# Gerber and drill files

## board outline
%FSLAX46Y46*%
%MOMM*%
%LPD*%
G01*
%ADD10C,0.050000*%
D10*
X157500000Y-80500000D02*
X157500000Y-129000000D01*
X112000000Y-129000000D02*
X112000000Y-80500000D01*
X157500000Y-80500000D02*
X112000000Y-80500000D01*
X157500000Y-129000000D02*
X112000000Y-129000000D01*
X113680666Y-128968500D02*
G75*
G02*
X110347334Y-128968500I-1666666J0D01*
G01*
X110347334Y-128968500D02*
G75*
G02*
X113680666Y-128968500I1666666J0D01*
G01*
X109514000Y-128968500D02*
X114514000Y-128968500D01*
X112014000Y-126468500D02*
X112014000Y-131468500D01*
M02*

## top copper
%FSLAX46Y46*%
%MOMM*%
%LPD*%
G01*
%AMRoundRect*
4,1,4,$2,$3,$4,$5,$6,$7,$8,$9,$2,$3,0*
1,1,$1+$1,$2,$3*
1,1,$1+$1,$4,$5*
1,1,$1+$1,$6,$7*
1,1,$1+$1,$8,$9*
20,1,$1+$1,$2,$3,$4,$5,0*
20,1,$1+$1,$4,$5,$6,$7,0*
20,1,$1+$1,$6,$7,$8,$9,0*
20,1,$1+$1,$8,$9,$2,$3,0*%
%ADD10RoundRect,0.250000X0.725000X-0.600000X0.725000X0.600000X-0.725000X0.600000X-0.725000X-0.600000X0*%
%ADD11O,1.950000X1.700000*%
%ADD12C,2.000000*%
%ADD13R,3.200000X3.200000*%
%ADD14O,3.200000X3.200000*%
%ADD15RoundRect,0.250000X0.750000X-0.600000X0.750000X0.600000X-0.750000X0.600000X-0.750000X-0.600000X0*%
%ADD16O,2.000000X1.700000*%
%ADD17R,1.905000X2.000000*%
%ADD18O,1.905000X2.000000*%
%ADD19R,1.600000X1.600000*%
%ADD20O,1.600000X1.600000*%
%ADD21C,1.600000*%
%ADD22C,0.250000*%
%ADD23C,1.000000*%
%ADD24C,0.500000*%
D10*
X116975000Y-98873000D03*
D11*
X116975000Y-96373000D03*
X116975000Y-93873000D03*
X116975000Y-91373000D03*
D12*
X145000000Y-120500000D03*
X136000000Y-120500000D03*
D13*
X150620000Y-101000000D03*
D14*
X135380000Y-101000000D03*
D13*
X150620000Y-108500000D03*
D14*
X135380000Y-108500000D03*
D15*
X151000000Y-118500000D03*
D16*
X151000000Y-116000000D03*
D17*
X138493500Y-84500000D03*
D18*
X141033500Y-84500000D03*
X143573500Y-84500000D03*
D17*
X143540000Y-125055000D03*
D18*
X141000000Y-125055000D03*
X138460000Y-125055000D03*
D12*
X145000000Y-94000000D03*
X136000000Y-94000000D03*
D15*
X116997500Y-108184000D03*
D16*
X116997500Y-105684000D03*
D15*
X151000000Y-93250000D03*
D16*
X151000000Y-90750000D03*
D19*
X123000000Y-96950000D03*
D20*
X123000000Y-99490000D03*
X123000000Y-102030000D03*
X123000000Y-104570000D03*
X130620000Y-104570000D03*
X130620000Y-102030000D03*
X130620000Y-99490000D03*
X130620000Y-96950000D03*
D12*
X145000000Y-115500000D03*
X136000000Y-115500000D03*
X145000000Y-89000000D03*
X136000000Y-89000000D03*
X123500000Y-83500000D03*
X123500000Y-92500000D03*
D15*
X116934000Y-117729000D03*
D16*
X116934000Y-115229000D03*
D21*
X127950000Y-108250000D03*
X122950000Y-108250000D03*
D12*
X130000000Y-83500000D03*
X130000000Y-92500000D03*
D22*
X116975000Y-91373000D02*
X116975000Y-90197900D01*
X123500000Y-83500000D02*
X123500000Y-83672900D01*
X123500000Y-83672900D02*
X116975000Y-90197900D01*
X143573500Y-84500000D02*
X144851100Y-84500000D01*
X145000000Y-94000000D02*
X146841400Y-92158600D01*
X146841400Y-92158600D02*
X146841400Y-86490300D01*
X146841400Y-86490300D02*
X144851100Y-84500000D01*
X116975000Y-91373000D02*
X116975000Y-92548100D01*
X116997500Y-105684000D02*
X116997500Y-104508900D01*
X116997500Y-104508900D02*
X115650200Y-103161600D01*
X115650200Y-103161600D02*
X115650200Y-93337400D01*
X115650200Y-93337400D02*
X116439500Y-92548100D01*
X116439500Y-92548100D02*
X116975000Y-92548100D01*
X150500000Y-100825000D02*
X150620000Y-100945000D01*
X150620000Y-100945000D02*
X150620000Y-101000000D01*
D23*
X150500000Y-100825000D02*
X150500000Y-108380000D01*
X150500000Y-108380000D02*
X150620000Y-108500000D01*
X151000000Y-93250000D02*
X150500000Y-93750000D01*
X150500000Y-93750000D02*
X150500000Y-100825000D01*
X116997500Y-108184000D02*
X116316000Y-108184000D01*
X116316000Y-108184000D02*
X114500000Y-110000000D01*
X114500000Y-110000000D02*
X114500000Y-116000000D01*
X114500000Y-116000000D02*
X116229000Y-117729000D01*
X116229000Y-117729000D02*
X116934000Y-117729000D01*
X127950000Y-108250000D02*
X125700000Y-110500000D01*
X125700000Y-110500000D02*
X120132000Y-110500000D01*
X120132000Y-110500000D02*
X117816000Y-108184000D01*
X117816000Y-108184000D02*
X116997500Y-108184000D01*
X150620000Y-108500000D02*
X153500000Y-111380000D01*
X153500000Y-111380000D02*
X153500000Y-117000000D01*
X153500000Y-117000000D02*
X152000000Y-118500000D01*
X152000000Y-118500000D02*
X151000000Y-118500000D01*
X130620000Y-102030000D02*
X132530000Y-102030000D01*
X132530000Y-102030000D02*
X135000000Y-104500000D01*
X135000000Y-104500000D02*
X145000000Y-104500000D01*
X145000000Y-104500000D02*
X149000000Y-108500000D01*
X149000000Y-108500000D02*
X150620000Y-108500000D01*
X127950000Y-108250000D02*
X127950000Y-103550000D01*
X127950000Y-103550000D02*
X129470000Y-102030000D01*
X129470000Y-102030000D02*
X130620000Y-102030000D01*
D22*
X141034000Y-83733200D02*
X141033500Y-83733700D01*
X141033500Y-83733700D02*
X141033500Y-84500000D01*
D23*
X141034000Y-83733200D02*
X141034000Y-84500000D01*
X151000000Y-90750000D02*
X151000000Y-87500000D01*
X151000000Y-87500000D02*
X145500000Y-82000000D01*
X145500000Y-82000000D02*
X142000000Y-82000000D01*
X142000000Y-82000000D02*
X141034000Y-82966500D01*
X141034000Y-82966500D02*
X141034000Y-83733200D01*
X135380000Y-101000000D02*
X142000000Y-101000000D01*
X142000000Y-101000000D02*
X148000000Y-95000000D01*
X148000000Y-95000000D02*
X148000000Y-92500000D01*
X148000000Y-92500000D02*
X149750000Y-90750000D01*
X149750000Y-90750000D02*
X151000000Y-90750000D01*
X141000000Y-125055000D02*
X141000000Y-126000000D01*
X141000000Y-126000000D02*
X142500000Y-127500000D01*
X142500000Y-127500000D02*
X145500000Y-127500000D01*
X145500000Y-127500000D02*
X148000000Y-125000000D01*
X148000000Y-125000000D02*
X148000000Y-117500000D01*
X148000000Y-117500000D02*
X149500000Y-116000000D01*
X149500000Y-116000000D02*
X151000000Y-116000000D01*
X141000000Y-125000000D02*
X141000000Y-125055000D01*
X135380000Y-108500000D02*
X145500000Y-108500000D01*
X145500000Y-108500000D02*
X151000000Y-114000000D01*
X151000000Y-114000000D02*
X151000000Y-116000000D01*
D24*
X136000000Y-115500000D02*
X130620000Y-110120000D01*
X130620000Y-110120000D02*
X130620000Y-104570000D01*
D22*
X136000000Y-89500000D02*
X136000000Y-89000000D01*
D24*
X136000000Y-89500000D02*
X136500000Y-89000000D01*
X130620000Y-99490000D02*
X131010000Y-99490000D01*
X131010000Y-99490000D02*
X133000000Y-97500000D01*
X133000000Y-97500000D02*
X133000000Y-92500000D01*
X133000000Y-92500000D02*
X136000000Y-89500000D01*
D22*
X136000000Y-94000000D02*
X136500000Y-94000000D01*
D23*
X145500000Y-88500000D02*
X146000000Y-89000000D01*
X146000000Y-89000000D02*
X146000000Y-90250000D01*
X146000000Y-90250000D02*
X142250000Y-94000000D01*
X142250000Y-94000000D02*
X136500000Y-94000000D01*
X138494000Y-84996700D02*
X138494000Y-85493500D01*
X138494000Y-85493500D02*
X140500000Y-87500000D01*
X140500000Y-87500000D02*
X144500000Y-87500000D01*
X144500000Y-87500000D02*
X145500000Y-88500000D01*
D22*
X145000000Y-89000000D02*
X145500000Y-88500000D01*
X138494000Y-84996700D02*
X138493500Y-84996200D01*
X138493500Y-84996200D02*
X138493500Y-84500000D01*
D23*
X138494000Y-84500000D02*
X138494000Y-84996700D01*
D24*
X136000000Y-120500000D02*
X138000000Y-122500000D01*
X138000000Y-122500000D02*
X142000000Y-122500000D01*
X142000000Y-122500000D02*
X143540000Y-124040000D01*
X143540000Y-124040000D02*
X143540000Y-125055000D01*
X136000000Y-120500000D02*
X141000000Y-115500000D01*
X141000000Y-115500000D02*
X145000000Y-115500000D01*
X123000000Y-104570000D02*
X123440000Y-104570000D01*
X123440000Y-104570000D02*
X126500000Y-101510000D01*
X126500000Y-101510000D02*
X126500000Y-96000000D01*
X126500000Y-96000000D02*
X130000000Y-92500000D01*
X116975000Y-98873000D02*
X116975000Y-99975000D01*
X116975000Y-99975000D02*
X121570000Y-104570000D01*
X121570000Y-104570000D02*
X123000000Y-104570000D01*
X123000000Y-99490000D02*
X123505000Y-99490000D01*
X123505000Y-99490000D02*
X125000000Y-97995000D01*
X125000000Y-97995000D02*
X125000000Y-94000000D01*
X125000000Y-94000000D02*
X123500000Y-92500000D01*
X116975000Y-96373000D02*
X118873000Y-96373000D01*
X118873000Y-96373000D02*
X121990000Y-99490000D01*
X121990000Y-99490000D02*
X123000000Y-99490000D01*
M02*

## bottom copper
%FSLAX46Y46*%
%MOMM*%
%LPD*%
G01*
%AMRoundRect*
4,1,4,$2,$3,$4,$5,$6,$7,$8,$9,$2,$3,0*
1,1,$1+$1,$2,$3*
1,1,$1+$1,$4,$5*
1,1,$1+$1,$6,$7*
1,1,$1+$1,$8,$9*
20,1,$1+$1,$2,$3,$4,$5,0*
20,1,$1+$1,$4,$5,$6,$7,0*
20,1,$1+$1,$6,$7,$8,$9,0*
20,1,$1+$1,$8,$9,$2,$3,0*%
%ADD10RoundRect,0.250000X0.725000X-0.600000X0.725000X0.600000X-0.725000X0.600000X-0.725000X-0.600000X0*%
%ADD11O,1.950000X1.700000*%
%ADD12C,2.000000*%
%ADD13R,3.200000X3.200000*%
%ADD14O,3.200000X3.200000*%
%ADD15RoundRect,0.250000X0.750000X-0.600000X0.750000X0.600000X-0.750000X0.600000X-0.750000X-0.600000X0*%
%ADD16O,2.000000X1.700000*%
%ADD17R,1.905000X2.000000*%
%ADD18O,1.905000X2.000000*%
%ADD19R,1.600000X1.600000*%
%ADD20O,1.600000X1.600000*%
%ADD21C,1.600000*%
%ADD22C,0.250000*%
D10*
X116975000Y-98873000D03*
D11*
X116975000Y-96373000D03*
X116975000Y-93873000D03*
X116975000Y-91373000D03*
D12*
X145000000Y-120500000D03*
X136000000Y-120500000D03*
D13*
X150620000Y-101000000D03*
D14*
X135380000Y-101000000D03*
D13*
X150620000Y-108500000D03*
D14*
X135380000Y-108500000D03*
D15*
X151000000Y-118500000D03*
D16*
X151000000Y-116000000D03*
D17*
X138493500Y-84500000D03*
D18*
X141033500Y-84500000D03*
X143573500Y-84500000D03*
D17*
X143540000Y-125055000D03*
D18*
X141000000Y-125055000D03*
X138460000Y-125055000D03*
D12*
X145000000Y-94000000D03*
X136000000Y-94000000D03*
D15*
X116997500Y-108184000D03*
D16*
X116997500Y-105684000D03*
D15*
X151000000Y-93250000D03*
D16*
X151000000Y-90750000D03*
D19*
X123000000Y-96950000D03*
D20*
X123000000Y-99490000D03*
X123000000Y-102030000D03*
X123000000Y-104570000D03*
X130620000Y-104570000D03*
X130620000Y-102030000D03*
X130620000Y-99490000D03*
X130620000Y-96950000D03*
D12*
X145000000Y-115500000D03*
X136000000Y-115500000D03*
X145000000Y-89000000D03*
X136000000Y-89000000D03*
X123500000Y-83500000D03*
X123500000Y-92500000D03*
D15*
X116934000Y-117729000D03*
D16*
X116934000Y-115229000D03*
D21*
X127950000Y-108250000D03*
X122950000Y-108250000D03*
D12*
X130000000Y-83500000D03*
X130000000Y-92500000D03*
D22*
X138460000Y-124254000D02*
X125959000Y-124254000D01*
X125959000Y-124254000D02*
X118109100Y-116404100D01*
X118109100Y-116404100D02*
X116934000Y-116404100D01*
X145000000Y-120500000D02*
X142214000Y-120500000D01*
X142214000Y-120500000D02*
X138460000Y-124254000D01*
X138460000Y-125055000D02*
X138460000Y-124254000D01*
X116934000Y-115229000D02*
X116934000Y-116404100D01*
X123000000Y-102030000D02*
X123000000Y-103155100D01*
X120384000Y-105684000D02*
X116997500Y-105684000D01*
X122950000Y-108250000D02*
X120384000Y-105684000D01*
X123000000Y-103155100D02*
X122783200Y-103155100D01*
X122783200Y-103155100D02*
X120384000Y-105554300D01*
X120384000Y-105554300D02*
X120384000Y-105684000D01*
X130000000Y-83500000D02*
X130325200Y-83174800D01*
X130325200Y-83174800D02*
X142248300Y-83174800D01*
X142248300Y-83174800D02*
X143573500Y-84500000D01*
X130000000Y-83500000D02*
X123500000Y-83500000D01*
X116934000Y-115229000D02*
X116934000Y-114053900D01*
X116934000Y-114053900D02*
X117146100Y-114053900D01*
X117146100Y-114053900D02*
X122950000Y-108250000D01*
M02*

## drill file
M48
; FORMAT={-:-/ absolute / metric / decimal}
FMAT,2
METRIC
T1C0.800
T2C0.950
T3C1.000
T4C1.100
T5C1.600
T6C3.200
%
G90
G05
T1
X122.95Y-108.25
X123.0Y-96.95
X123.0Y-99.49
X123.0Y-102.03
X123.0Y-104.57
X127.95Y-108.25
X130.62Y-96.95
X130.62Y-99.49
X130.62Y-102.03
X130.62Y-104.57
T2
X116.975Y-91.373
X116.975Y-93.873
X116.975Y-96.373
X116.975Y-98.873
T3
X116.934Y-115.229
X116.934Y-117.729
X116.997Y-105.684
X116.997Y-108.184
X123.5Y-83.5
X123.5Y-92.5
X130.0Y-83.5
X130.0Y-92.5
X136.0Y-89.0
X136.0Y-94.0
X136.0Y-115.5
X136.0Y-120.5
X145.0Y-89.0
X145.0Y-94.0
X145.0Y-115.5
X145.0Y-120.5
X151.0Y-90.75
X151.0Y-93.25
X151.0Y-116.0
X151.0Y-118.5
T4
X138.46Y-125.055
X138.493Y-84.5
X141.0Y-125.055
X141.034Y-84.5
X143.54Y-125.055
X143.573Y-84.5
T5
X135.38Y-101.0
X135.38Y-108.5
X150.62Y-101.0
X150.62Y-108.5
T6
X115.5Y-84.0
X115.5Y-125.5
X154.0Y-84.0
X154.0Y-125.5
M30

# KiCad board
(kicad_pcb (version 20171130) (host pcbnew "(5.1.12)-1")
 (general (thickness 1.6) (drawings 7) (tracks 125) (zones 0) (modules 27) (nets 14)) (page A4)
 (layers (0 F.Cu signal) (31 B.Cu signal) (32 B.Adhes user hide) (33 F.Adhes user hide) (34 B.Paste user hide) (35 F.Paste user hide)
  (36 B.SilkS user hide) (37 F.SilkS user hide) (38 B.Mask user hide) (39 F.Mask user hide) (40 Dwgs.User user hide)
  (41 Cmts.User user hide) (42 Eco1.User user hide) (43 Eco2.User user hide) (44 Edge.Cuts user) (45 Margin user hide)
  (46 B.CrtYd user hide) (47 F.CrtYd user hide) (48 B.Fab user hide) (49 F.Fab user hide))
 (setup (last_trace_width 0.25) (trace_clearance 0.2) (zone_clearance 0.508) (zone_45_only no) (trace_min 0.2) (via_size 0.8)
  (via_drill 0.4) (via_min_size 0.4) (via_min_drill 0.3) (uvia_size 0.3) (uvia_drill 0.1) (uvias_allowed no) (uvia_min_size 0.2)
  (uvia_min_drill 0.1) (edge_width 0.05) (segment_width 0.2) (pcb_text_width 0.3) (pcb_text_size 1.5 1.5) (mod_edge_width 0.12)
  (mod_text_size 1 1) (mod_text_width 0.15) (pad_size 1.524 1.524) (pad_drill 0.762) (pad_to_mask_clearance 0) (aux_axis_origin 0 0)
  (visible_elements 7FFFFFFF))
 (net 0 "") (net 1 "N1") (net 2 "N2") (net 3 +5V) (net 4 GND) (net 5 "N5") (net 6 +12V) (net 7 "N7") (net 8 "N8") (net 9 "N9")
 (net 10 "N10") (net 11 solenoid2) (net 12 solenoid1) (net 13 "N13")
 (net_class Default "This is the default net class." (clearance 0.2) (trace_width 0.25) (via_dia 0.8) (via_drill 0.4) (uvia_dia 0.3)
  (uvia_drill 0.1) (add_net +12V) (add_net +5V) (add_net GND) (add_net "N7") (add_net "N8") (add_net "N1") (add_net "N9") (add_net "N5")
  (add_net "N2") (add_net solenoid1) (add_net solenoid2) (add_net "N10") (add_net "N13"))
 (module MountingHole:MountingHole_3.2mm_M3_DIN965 (layer F.Cu) (at 115.5 84)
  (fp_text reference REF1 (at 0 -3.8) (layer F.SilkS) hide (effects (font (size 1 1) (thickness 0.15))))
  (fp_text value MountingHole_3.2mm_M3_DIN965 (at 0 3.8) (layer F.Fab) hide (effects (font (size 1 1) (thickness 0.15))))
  (pad "" np_thru_hole circle (at 0 0) (size 3.2 3.2) (drill 3.2) (layers *.Cu *.Mask)))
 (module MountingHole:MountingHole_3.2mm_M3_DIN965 (layer F.Cu) (at 115.5 125.5)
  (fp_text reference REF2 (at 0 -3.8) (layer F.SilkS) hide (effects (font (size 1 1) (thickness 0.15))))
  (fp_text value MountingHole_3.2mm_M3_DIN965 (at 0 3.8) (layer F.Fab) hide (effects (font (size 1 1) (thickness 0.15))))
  (pad "" np_thru_hole circle (at 0 0) (size 3.2 3.2) (drill 3.2) (layers *.Cu *.Mask)))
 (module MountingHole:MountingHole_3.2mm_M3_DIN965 (layer F.Cu) (at 154 84)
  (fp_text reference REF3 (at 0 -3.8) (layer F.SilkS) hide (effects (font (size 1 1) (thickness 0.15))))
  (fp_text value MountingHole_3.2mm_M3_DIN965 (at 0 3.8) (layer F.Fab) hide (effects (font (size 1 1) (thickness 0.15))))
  (pad "" np_thru_hole circle (at 0 0) (size 3.2 3.2) (drill 3.2) (layers *.Cu *.Mask)))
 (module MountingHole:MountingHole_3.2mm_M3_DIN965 (layer F.Cu) (at 154 125.5)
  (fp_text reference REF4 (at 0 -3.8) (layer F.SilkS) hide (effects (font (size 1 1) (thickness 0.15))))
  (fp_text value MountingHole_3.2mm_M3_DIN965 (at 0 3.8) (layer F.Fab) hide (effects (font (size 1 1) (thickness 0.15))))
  (pad "" np_thru_hole circle (at 0 0) (size 3.2 3.2) (drill 3.2) (layers *.Cu *.Mask)))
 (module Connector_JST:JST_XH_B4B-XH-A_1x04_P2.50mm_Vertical (layer F.Cu) (at 116.975 98.873 90)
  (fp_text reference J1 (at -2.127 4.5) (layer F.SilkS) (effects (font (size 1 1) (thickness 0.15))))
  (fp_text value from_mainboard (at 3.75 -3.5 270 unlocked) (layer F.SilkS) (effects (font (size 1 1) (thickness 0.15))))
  (pad 1 thru_hole roundrect (at 0 0 90) (size 1.7 1.95) (drill 0.95) (layers *.Cu *.Mask) (roundrect_rratio 0.1470588235) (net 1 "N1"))
  (pad 2 thru_hole oval (at 2.5 0 90) (size 1.7 1.95) (drill 0.95) (layers *.Cu *.Mask) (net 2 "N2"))
  (pad 3 thru_hole oval (at 5 0 90) (size 1.7 1.95) (drill 0.95) (layers *.Cu *.Mask) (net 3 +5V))
  (pad 4 thru_hole oval (at 7.5 0 90) (size 1.7 1.95) (drill 0.95) (layers *.Cu *.Mask) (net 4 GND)))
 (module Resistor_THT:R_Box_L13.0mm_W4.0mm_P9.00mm (layer F.Cu) (at 145 120.5 180)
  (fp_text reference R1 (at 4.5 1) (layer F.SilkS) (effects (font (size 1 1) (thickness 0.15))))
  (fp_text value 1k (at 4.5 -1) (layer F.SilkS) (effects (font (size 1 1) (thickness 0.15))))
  (pad 1 thru_hole circle (at 0 0 180) (size 2 2) (drill 1) (layers *.Cu *.Mask) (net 4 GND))
  (pad 2 thru_hole circle (at 9 0 180) (size 2 2) (drill 1) (layers *.Cu *.Mask) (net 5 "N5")))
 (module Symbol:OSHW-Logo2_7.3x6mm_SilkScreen (layer F.Cu) (at 125 113.5 90)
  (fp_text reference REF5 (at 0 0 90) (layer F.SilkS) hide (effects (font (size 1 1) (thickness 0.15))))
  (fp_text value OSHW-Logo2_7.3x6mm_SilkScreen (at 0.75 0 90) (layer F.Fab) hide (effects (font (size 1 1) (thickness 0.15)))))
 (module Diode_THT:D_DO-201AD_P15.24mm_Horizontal (layer F.Cu) (at 150.62 101 180)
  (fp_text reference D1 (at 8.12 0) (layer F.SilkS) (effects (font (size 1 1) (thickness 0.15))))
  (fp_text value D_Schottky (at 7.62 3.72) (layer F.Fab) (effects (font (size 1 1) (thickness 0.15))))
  (pad 1 thru_hole rect (at 0 0 180) (size 3.2 3.2) (drill 1.6) (layers *.Cu *.Mask) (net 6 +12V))
  (pad 2 thru_hole oval (at 15.24 0 180) (size 3.2 3.2) (drill 1.6) (layers *.Cu *.Mask) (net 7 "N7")))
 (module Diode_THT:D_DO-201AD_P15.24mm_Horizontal (layer F.Cu) (at 150.62 108.5 180)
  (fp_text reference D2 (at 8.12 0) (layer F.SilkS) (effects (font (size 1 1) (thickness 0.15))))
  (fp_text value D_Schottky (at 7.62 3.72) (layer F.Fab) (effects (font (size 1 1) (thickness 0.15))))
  (pad 1 thru_hole rect (at 0 0 180) (size 3.2 3.2) (drill 1.6) (layers *.Cu *.Mask) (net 6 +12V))
  (pad 2 thru_hole oval (at 15.24 0 180) (size 3.2 3.2) (drill 1.6) (layers *.Cu *.Mask) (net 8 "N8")))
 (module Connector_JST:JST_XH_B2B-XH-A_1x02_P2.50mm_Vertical (layer F.Cu) (at 151 118.5 90)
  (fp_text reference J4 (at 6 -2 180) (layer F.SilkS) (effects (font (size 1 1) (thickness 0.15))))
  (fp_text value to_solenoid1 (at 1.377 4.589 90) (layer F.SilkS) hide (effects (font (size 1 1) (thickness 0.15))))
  (pad 1 thru_hole roundrect (at 0 0 90) (size 1.7 2) (drill 1) (layers *.Cu *.Mask) (roundrect_rratio 0.1470588235) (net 6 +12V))
  (pad 2 thru_hole oval (at 2.5 0 90) (size 1.7 2) (drill 1) (layers *.Cu *.Mask) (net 8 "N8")))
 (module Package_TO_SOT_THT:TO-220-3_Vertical (layer F.Cu) (at 138.4935 84.5)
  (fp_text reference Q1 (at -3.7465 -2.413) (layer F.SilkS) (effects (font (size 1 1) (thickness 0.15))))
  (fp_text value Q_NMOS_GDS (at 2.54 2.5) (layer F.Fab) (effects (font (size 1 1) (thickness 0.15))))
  (pad 1 thru_hole rect (at 0 0) (size 1.905 2) (drill 1.1) (layers *.Cu *.Mask) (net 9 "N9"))
  (pad 2 thru_hole oval (at 2.54 0) (size 1.905 2) (drill 1.1) (layers *.Cu *.Mask) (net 7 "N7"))
  (pad 3 thru_hole oval (at 5.08 0) (size 1.905 2) (drill 1.1) (layers *.Cu *.Mask) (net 4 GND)))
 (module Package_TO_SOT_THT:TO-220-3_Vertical (layer F.Cu) (at 143.54 125.055 180)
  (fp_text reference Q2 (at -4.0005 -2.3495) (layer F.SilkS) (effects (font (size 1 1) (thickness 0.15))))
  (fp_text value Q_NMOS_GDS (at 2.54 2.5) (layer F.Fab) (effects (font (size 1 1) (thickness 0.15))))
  (pad 1 thru_hole rect (at 0 0 180) (size 1.905 2) (drill 1.1) (layers *.Cu *.Mask) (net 5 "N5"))
  (pad 2 thru_hole oval (at 2.54 0 180) (size 1.905 2) (drill 1.1) (layers *.Cu *.Mask) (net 8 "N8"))
  (pad 3 thru_hole oval (at 5.08 0 180) (size 1.905 2) (drill 1.1) (layers *.Cu *.Mask) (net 4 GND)))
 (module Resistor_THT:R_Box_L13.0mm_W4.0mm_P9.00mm (layer F.Cu) (at 145 94 180)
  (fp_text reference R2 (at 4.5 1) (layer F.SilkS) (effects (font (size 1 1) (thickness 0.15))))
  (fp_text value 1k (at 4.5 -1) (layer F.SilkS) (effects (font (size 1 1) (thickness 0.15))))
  (pad 1 thru_hole circle (at 0 0 180) (size 2 2) (drill 1) (layers *.Cu *.Mask) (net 4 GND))
  (pad 2 thru_hole circle (at 9 0 180) (size 2 2) (drill 1) (layers *.Cu *.Mask) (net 9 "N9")))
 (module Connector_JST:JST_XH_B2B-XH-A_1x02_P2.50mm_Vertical (layer F.Cu) (at 116.9975 108.184 90)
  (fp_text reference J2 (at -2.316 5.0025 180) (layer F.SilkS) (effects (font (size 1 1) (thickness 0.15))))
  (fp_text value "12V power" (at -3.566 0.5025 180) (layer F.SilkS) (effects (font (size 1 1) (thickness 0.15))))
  (pad 1 thru_hole roundrect (at 0 0 90) (size 1.7 2) (drill 1) (layers *.Cu *.Mask) (roundrect_rratio 0.1470588235) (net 6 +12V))
  (pad 2 thru_hole oval (at 2.5 0 90) (size 1.7 2) (drill 1) (layers *.Cu *.Mask) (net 4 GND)))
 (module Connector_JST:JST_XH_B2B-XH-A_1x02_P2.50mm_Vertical (layer F.Cu) (at 151 93.25 90)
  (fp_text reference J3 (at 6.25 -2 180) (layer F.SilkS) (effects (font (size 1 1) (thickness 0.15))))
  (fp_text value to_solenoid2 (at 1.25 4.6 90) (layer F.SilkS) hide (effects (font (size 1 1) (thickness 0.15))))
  (pad 1 thru_hole roundrect (at 0 0 90) (size 1.7 2) (drill 1) (layers *.Cu *.Mask) (roundrect_rratio 0.1470588235) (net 6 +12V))
  (pad 2 thru_hole oval (at 2.5 0 90) (size 1.7 2) (drill 1) (layers *.Cu *.Mask) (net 7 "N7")))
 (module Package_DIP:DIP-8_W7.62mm (layer F.Cu) (at 123 96.95)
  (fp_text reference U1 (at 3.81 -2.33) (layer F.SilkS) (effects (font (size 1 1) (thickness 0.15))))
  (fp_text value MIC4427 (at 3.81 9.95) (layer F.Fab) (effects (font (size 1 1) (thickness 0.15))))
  (pad 1 thru_hole rect (at 0 0) (size 1.6 1.6) (drill 0.8) (layers *.Cu *.Mask) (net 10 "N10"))
  (pad 2 thru_hole oval (at 0 2.54) (size 1.6 1.6) (drill 0.8) (layers *.Cu *.Mask) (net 2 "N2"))
  (pad 3 thru_hole oval (at 0 5.08) (size 1.6 1.6) (drill 0.8) (layers *.Cu *.Mask) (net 4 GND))
  (pad 4 thru_hole oval (at 0 7.62) (size 1.6 1.6) (drill 0.8) (layers *.Cu *.Mask) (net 1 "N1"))
  (pad 5 thru_hole oval (at 7.62 7.62) (size 1.6 1.6) (drill 0.8) (layers *.Cu *.Mask) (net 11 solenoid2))
  (pad 6 thru_hole oval (at 7.62 5.08) (size 1.6 1.6) (drill 0.8) (layers *.Cu *.Mask) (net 6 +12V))
  (pad 7 thru_hole oval (at 7.62 2.54) (size 1.6 1.6) (drill 0.8) (layers *.Cu *.Mask) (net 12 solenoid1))
  (pad 8 thru_hole oval (at 7.62 0) (size 1.6 1.6) (drill 0.8) (layers *.Cu *.Mask) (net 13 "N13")))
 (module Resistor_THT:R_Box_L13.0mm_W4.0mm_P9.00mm (layer F.Cu) (at 145 115.5 180)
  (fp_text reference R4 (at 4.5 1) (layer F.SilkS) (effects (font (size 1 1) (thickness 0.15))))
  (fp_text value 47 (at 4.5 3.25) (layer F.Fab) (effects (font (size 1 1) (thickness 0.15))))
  (pad 1 thru_hole circle (at 0 0 180) (size 2 2) (drill 1) (layers *.Cu *.Mask) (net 5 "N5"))
  (pad 2 thru_hole circle (at 9 0 180) (size 2 2) (drill 1) (layers *.Cu *.Mask) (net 11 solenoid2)))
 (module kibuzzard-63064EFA (layer F.Cu) (at 113.5 116.479 90)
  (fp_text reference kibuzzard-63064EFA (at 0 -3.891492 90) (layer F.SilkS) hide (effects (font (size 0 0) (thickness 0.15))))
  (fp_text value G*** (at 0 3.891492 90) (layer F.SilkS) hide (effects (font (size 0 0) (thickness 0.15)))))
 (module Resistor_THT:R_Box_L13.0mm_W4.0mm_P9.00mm (layer F.Cu) (at 145 89 180)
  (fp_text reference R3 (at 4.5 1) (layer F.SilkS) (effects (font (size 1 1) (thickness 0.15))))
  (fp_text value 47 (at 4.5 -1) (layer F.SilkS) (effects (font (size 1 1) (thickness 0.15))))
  (pad 1 thru_hole circle (at 0 0 180) (size 2 2) (drill 1) (layers *.Cu *.Mask) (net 9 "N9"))
  (pad 2 thru_hole circle (at 9 0 180) (size 2 2) (drill 1) (layers *.Cu *.Mask) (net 12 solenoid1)))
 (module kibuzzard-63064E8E (layer F.Cu) (at 156 92 90)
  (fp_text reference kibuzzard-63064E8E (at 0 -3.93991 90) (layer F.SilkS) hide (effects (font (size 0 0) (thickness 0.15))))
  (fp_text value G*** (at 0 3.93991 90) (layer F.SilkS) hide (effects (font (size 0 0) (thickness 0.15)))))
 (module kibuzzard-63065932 (layer F.Cu) (at 113.5 107 90)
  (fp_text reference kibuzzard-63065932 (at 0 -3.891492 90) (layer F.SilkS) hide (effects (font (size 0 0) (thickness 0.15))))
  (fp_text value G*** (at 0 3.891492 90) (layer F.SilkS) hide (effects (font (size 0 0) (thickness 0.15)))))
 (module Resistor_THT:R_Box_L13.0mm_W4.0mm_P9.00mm (layer F.Cu) (at 123.5 83.5 270)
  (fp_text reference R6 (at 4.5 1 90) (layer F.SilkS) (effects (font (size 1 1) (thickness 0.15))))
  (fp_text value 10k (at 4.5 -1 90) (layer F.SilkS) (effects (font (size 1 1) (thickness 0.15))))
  (pad 1 thru_hole circle (at 0 0 270) (size 2 2) (drill 1) (layers *.Cu *.Mask) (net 4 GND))
  (pad 2 thru_hole circle (at 9 0 270) (size 2 2) (drill 1) (layers *.Cu *.Mask) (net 2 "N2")))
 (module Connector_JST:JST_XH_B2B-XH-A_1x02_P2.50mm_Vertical (layer F.Cu) (at 116.934 117.729 90)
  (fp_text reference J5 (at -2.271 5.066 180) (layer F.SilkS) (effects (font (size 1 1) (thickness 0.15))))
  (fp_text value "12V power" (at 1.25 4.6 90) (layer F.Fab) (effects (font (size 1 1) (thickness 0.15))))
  (pad 1 thru_hole roundrect (at 0 0 90) (size 1.7 2) (drill 1) (layers *.Cu *.Mask) (roundrect_rratio 0.1470588235) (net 6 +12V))
  (pad 2 thru_hole oval (at 2.5 0 90) (size 1.7 2) (drill 1) (layers *.Cu *.Mask) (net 4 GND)))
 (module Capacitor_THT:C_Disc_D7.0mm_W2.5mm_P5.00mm (layer F.Cu) (at 127.95 108.25 180)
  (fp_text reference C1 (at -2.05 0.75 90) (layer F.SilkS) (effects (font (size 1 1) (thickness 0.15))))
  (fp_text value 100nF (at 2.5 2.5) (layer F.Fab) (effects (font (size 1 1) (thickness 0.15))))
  (pad 1 thru_hole circle (at 0 0 180) (size 1.6 1.6) (drill 0.8) (layers *.Cu *.Mask) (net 6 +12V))
  (pad 2 thru_hole circle (at 5 0 180) (size 1.6 1.6) (drill 0.8) (layers *.Cu *.Mask) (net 4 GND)))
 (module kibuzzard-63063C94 (layer F.Cu) (at 156 117.5 90)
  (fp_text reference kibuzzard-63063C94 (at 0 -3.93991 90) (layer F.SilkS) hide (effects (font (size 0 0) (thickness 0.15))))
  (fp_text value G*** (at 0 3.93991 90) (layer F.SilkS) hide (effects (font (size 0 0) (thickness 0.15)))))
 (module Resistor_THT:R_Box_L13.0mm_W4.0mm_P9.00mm (layer F.Cu) (at 130 83.5 270)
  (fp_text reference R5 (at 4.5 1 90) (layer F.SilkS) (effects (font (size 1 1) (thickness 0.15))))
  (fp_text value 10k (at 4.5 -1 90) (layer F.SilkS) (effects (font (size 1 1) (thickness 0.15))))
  (pad 1 thru_hole circle (at 0 0 270) (size 2 2) (drill 1) (layers *.Cu *.Mask) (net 4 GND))
  (pad 2 thru_hole circle (at 9 0 270) (size 2 2) (drill 1) (layers *.Cu *.Mask) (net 1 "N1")))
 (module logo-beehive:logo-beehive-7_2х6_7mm (layer F.Cu) (at 123 124.5)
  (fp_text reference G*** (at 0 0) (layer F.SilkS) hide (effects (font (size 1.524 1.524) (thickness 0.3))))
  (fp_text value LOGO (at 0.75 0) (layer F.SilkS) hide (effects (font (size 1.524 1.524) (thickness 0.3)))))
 (gr_line (start 157.5 80.5) (end 157.5 129) (layer Edge.Cuts) (width 0.05))
 (gr_line (start 112 129) (end 112 80.5) (layer Edge.Cuts) (width 0.05))
 (gr_line (start 157.5 80.5) (end 112 80.5) (layer Edge.Cuts) (width 0.05))
 (gr_line (start 157.5 129) (end 112 129) (layer Edge.Cuts) (width 0.05))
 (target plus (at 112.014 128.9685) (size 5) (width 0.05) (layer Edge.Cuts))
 (segment (start 138.46 124.254) (end 125.959 124.254) (width 0.25) (layer B.Cu) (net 4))
 (segment (start 125.959 124.254) (end 118.1091 116.4041) (width 0.25) (layer B.Cu) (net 4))
 (segment (start 118.1091 116.4041) (end 116.934 116.4041) (width 0.25) (layer B.Cu) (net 4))
 (segment (start 145 120.5) (end 142.214 120.5) (width 0.25) (layer B.Cu) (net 4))
 (segment (start 142.214 120.5) (end 138.46 124.254) (width 0.25) (layer B.Cu) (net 4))
 (segment (start 138.46 125.055) (end 138.46 124.254) (width 0.25) (layer B.Cu) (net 4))
 (segment (start 116.934 115.229) (end 116.934 116.4041) (width 0.25) (layer B.Cu) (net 4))
 (segment (start 116.975 91.373) (end 116.975 90.1979) (width 0.25) (layer F.Cu) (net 4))
 (segment (start 123.5 83.5) (end 123.5 83.6729) (width 0.25) (layer F.Cu) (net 4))
 (segment (start 123.5 83.6729) (end 116.975 90.1979) (width 0.25) (layer F.Cu) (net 4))
 (segment (start 143.5735 84.5) (end 144.8511 84.5) (width 0.25) (layer F.Cu) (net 4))
 (segment (start 145 94) (end 146.8414 92.1586) (width 0.25) (layer F.Cu) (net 4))
 (segment (start 146.8414 92.1586) (end 146.8414 86.4903) (width 0.25) (layer F.Cu) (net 4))
 (segment (start 146.8414 86.4903) (end 144.8511 84.5) (width 0.25) (layer F.Cu) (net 4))
 (segment (start 116.975 91.373) (end 116.975 92.5481) (width 0.25) (layer F.Cu) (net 4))
 (segment (start 116.9975 105.684) (end 116.9975 104.5089) (width 0.25) (layer F.Cu) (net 4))
 (segment (start 116.9975 104.5089) (end 115.6502 103.1616) (width 0.25) (layer F.Cu) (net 4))
 (segment (start 115.6502 103.1616) (end 115.6502 93.3374) (width 0.25) (layer F.Cu) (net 4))
 (segment (start 115.6502 93.3374) (end 116.4395 92.5481) (width 0.25) (layer F.Cu) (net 4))
 (segment (start 116.4395 92.5481) (end 116.975 92.5481) (width 0.25) (layer F.Cu) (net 4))
 (segment (start 123 102.03) (end 123 103.1551) (width 0.25) (layer B.Cu) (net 4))
 (segment (start 120.384 105.684) (end 116.9975 105.684) (width 0.25) (layer B.Cu) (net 4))
 (segment (start 122.95 108.25) (end 120.384 105.684) (width 0.25) (layer B.Cu) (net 4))
 (segment (start 123 103.1551) (end 122.7832 103.1551) (width 0.25) (layer B.Cu) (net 4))
 (segment (start 122.7832 103.1551) (end 120.384 105.5543) (width 0.25) (layer B.Cu) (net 4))
 (segment (start 120.384 105.5543) (end 120.384 105.684) (width 0.25) (layer B.Cu) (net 4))
 (segment (start 130 83.5) (end 130.3252 83.1748) (width 0.25) (layer B.Cu) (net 4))
 (segment (start 130.3252 83.1748) (end 142.2483 83.1748) (width 0.25) (layer B.Cu) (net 4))
 (segment (start 142.2483 83.1748) (end 143.5735 84.5) (width 0.25) (layer B.Cu) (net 4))
 (segment (start 130 83.5) (end 123.5 83.5) (width 0.25) (layer B.Cu) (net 4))
 (segment (start 116.934 115.229) (end 116.934 114.0539) (width 0.25) (layer B.Cu) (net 4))
 (segment (start 116.934 114.0539) (end 117.1461 114.0539) (width 0.25) (layer B.Cu) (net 4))
 (segment (start 117.1461 114.0539) (end 122.95 108.25) (width 0.25) (layer B.Cu) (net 4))
 (segment (start 150.5 100.825) (end 150.62 100.945) (width 0.25) (layer F.Cu) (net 6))
 (segment (start 150.62 100.945) (end 150.62 101) (width 0.25) (layer F.Cu) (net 6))
 (segment (start 150.5 100.825) (end 150.5 108.38) (width 1) (layer F.Cu) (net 6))
 (segment (start 150.5 108.38) (end 150.62 108.5) (width 1) (layer F.Cu) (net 6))
 (segment (start 151 93.25) (end 150.5 93.75) (width 1) (layer F.Cu) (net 6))
 (segment (start 150.5 93.75) (end 150.5 100.825) (width 1) (layer F.Cu) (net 6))
 (segment (start 116.9975 108.184) (end 116.316 108.184) (width 1) (layer F.Cu) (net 6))
 (segment (start 116.316 108.184) (end 114.5 110) (width 1) (layer F.Cu) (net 6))
 (segment (start 114.5 110) (end 114.5 116) (width 1) (layer F.Cu) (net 6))
 (segment (start 114.5 116) (end 116.229 117.729) (width 1) (layer F.Cu) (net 6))
 (segment (start 116.229 117.729) (end 116.934 117.729) (width 1) (layer F.Cu) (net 6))
 (segment (start 127.95 108.25) (end 125.7 110.5) (width 1) (layer F.Cu) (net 6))
 (segment (start 125.7 110.5) (end 120.132 110.5) (width 1) (layer F.Cu) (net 6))
 (segment (start 120.132 110.5) (end 117.816 108.184) (width 1) (layer F.Cu) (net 6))
 (segment (start 117.816 108.184) (end 116.9975 108.184) (width 1) (layer F.Cu) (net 6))
 (segment (start 150.62 108.5) (end 153.5 111.38) (width 1) (layer F.Cu) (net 6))
 (segment (start 153.5 111.38) (end 153.5 117) (width 1) (layer F.Cu) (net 6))
 (segment (start 153.5 117) (end 152 118.5) (width 1) (layer F.Cu) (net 6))
 (segment (start 152 118.5) (end 151 118.5) (width 1) (layer F.Cu) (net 6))
 (segment (start 130.62 102.03) (end 132.53 102.03) (width 1) (layer F.Cu) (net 6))
 (segment (start 132.53 102.03) (end 135 104.5) (width 1) (layer F.Cu) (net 6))
 (segment (start 135 104.5) (end 145 104.5) (width 1) (layer F.Cu) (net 6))
 (segment (start 145 104.5) (end 149 108.5) (width 1) (layer F.Cu) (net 6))
 (segment (start 149 108.5) (end 150.62 108.5) (width 1) (layer F.Cu) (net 6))
 (segment (start 127.95 108.25) (end 127.95 103.55) (width 1) (layer F.Cu) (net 6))
 (segment (start 127.95 103.55) (end 129.47 102.03) (width 1) (layer F.Cu) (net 6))
 (segment (start 129.47 102.03) (end 130.62 102.03) (width 1) (layer F.Cu) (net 6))
 (segment (start 141.034 83.7332) (end 141.0335 83.7337) (width 0.25) (layer F.Cu) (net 7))
 (segment (start 141.0335 83.7337) (end 141.0335 84.5) (width 0.25) (layer F.Cu) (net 7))
 (segment (start 141.034 83.7332) (end 141.034 84.5) (width 1) (layer F.Cu) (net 7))
 (segment (start 151 90.75) (end 151 87.5) (width 1) (layer F.Cu) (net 7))
 (segment (start 151 87.5) (end 145.5 82) (width 1) (layer F.Cu) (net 7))
 (segment (start 145.5 82) (end 142 82) (width 1) (layer F.Cu) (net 7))
 (segment (start 142 82) (end 141.034 82.9665) (width 1) (layer F.Cu) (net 7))
 (segment (start 141.034 82.9665) (end 141.034 83.7332) (width 1) (layer F.Cu) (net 7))
 (segment (start 135.38 101) (end 142 101) (width 1) (layer F.Cu) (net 7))
 (segment (start 142 101) (end 148 95) (width 1) (layer F.Cu) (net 7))
 (segment (start 148 95) (end 148 92.5) (width 1) (layer F.Cu) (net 7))
 (segment (start 148 92.5) (end 149.75 90.75) (width 1) (layer F.Cu) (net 7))
 (segment (start 149.75 90.75) (end 151 90.75) (width 1) (layer F.Cu) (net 7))
 (segment (start 141 125.055) (end 141 126) (width 1) (layer F.Cu) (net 8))
 (segment (start 141 126) (end 142.5 127.5) (width 1) (layer F.Cu) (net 8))
 (segment (start 142.5 127.5) (end 145.5 127.5) (width 1) (layer F.Cu) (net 8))
 (segment (start 145.5 127.5) (end 148 125) (width 1) (layer F.Cu) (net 8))
 (segment (start 148 125) (end 148 117.5) (width 1) (layer F.Cu) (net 8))
 (segment (start 148 117.5) (end 149.5 116) (width 1) (layer F.Cu) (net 8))
 (segment (start 149.5 116) (end 151 116) (width 1) (layer F.Cu) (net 8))
 (segment (start 141 125) (end 141 125.055) (width 1) (layer F.Cu) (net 8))
 (segment (start 135.38 108.5) (end 145.5 108.5) (width 1) (layer F.Cu) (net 8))
 (segment (start 145.5 108.5) (end 151 114) (width 1) (layer F.Cu) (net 8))
 (segment (start 151 114) (end 151 116) (width 1) (layer F.Cu) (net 8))
 (segment (start 136 115.5) (end 130.62 110.12) (width 0.5) (layer F.Cu) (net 11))
 (segment (start 130.62 110.12) (end 130.62 104.57) (width 0.5) (layer F.Cu) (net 11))
 (segment (start 136 89.5) (end 136 89) (width 0.25) (layer F.Cu) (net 12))
 (segment (start 136 89.5) (end 136.5 89) (width 0.5) (layer F.Cu) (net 12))
 (segment (start 130.62 99.49) (end 131.01 99.49) (width 0.5) (layer F.Cu) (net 12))
 (segment (start 131.01 99.49) (end 133 97.5) (width 0.5) (layer F.Cu) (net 12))
 (segment (start 133 97.5) (end 133 92.5) (width 0.5) (layer F.Cu) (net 12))
 (segment (start 133 92.5) (end 136 89.5) (width 0.5) (layer F.Cu) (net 12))
 (segment (start 136 94) (end 136.5 94) (width 0.25) (layer F.Cu) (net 9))
 (segment (start 145.5 88.5) (end 146 89) (width 1) (layer F.Cu) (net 9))
 (segment (start 146 89) (end 146 90.25) (width 1) (layer F.Cu) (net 9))
 (segment (start 146 90.25) (end 142.25 94) (width 1) (layer F.Cu) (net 9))
 (segment (start 142.25 94) (end 136.5 94) (width 1) (layer F.Cu) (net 9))
 (segment (start 138.494 84.9967) (end 138.494 85.4935) (width 1) (layer F.Cu) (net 9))
 (segment (start 138.494 85.4935) (end 140.5 87.5) (width 1) (layer F.Cu) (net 9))
 (segment (start 140.5 87.5) (end 144.5 87.5) (width 1) (layer F.Cu) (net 9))
 (segment (start 144.5 87.5) (end 145.5 88.5) (width 1) (layer F.Cu) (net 9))
 (segment (start 145 89) (end 145.5 88.5) (width 0.25) (layer F.Cu) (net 9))
 (segment (start 138.494 84.9967) (end 138.4935 84.9962) (width 0.25) (layer F.Cu) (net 9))
 (segment (start 138.4935 84.9962) (end 138.4935 84.5) (width 0.25) (layer F.Cu) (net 9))
 (segment (start 138.494 84.5) (end 138.494 84.9967) (width 1) (layer F.Cu) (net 9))
 (segment (start 136 120.5) (end 138 122.5) (width 0.5) (layer F.Cu) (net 5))
 (segment (start 138 122.5) (end 142 122.5) (width 0.5) (layer F.Cu) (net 5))
 (segment (start 142 122.5) (end 143.54 124.04) (width 0.5) (layer F.Cu) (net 5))
 (segment (start 143.54 124.04) (end 143.54 125.055) (width 0.5) (layer F.Cu) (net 5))
 (segment (start 136 120.5) (end 141 115.5) (width 0.5) (layer F.Cu) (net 5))
 (segment (start 141 115.5) (end 145 115.5) (width 0.5) (layer F.Cu) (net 5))
 (segment (start 123 104.57) (end 123.44 104.57) (width 0.5) (layer F.Cu) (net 1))
 (segment (start 123.44 104.57) (end 126.5 101.51) (width 0.5) (layer F.Cu) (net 1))
 (segment (start 126.5 101.51) (end 126.5 96) (width 0.5) (layer F.Cu) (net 1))
 (segment (start 126.5 96) (end 130 92.5) (width 0.5) (layer F.Cu) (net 1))
 (segment (start 116.975 98.873) (end 116.975 99.975) (width 0.5) (layer F.Cu) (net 1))
 (segment (start 116.975 99.975) (end 121.57 104.57) (width 0.5) (layer F.Cu) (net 1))
 (segment (start 121.57 104.57) (end 123 104.57) (width 0.5) (layer F.Cu) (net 1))
 (segment (start 123 99.49) (end 123.505 99.49) (width 0.5) (layer F.Cu) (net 2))
 (segment (start 123.505 99.49) (end 125 97.995) (width 0.5) (layer F.Cu) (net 2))
 (segment (start 125 97.995) (end 125 94) (width 0.5) (layer F.Cu) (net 2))
 (segment (start 125 94) (end 123.5 92.5) (width 0.5) (layer F.Cu) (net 2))
 (segment (start 116.975 96.373) (end 118.873 96.373) (width 0.5) (layer F.Cu) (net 2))
 (segment (start 118.873 96.373) (end 121.99 99.49) (width 0.5) (layer F.Cu) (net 2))
 (segment (start 121.99 99.49) (end 123 99.49) (width 0.5) (layer F.Cu) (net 2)))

